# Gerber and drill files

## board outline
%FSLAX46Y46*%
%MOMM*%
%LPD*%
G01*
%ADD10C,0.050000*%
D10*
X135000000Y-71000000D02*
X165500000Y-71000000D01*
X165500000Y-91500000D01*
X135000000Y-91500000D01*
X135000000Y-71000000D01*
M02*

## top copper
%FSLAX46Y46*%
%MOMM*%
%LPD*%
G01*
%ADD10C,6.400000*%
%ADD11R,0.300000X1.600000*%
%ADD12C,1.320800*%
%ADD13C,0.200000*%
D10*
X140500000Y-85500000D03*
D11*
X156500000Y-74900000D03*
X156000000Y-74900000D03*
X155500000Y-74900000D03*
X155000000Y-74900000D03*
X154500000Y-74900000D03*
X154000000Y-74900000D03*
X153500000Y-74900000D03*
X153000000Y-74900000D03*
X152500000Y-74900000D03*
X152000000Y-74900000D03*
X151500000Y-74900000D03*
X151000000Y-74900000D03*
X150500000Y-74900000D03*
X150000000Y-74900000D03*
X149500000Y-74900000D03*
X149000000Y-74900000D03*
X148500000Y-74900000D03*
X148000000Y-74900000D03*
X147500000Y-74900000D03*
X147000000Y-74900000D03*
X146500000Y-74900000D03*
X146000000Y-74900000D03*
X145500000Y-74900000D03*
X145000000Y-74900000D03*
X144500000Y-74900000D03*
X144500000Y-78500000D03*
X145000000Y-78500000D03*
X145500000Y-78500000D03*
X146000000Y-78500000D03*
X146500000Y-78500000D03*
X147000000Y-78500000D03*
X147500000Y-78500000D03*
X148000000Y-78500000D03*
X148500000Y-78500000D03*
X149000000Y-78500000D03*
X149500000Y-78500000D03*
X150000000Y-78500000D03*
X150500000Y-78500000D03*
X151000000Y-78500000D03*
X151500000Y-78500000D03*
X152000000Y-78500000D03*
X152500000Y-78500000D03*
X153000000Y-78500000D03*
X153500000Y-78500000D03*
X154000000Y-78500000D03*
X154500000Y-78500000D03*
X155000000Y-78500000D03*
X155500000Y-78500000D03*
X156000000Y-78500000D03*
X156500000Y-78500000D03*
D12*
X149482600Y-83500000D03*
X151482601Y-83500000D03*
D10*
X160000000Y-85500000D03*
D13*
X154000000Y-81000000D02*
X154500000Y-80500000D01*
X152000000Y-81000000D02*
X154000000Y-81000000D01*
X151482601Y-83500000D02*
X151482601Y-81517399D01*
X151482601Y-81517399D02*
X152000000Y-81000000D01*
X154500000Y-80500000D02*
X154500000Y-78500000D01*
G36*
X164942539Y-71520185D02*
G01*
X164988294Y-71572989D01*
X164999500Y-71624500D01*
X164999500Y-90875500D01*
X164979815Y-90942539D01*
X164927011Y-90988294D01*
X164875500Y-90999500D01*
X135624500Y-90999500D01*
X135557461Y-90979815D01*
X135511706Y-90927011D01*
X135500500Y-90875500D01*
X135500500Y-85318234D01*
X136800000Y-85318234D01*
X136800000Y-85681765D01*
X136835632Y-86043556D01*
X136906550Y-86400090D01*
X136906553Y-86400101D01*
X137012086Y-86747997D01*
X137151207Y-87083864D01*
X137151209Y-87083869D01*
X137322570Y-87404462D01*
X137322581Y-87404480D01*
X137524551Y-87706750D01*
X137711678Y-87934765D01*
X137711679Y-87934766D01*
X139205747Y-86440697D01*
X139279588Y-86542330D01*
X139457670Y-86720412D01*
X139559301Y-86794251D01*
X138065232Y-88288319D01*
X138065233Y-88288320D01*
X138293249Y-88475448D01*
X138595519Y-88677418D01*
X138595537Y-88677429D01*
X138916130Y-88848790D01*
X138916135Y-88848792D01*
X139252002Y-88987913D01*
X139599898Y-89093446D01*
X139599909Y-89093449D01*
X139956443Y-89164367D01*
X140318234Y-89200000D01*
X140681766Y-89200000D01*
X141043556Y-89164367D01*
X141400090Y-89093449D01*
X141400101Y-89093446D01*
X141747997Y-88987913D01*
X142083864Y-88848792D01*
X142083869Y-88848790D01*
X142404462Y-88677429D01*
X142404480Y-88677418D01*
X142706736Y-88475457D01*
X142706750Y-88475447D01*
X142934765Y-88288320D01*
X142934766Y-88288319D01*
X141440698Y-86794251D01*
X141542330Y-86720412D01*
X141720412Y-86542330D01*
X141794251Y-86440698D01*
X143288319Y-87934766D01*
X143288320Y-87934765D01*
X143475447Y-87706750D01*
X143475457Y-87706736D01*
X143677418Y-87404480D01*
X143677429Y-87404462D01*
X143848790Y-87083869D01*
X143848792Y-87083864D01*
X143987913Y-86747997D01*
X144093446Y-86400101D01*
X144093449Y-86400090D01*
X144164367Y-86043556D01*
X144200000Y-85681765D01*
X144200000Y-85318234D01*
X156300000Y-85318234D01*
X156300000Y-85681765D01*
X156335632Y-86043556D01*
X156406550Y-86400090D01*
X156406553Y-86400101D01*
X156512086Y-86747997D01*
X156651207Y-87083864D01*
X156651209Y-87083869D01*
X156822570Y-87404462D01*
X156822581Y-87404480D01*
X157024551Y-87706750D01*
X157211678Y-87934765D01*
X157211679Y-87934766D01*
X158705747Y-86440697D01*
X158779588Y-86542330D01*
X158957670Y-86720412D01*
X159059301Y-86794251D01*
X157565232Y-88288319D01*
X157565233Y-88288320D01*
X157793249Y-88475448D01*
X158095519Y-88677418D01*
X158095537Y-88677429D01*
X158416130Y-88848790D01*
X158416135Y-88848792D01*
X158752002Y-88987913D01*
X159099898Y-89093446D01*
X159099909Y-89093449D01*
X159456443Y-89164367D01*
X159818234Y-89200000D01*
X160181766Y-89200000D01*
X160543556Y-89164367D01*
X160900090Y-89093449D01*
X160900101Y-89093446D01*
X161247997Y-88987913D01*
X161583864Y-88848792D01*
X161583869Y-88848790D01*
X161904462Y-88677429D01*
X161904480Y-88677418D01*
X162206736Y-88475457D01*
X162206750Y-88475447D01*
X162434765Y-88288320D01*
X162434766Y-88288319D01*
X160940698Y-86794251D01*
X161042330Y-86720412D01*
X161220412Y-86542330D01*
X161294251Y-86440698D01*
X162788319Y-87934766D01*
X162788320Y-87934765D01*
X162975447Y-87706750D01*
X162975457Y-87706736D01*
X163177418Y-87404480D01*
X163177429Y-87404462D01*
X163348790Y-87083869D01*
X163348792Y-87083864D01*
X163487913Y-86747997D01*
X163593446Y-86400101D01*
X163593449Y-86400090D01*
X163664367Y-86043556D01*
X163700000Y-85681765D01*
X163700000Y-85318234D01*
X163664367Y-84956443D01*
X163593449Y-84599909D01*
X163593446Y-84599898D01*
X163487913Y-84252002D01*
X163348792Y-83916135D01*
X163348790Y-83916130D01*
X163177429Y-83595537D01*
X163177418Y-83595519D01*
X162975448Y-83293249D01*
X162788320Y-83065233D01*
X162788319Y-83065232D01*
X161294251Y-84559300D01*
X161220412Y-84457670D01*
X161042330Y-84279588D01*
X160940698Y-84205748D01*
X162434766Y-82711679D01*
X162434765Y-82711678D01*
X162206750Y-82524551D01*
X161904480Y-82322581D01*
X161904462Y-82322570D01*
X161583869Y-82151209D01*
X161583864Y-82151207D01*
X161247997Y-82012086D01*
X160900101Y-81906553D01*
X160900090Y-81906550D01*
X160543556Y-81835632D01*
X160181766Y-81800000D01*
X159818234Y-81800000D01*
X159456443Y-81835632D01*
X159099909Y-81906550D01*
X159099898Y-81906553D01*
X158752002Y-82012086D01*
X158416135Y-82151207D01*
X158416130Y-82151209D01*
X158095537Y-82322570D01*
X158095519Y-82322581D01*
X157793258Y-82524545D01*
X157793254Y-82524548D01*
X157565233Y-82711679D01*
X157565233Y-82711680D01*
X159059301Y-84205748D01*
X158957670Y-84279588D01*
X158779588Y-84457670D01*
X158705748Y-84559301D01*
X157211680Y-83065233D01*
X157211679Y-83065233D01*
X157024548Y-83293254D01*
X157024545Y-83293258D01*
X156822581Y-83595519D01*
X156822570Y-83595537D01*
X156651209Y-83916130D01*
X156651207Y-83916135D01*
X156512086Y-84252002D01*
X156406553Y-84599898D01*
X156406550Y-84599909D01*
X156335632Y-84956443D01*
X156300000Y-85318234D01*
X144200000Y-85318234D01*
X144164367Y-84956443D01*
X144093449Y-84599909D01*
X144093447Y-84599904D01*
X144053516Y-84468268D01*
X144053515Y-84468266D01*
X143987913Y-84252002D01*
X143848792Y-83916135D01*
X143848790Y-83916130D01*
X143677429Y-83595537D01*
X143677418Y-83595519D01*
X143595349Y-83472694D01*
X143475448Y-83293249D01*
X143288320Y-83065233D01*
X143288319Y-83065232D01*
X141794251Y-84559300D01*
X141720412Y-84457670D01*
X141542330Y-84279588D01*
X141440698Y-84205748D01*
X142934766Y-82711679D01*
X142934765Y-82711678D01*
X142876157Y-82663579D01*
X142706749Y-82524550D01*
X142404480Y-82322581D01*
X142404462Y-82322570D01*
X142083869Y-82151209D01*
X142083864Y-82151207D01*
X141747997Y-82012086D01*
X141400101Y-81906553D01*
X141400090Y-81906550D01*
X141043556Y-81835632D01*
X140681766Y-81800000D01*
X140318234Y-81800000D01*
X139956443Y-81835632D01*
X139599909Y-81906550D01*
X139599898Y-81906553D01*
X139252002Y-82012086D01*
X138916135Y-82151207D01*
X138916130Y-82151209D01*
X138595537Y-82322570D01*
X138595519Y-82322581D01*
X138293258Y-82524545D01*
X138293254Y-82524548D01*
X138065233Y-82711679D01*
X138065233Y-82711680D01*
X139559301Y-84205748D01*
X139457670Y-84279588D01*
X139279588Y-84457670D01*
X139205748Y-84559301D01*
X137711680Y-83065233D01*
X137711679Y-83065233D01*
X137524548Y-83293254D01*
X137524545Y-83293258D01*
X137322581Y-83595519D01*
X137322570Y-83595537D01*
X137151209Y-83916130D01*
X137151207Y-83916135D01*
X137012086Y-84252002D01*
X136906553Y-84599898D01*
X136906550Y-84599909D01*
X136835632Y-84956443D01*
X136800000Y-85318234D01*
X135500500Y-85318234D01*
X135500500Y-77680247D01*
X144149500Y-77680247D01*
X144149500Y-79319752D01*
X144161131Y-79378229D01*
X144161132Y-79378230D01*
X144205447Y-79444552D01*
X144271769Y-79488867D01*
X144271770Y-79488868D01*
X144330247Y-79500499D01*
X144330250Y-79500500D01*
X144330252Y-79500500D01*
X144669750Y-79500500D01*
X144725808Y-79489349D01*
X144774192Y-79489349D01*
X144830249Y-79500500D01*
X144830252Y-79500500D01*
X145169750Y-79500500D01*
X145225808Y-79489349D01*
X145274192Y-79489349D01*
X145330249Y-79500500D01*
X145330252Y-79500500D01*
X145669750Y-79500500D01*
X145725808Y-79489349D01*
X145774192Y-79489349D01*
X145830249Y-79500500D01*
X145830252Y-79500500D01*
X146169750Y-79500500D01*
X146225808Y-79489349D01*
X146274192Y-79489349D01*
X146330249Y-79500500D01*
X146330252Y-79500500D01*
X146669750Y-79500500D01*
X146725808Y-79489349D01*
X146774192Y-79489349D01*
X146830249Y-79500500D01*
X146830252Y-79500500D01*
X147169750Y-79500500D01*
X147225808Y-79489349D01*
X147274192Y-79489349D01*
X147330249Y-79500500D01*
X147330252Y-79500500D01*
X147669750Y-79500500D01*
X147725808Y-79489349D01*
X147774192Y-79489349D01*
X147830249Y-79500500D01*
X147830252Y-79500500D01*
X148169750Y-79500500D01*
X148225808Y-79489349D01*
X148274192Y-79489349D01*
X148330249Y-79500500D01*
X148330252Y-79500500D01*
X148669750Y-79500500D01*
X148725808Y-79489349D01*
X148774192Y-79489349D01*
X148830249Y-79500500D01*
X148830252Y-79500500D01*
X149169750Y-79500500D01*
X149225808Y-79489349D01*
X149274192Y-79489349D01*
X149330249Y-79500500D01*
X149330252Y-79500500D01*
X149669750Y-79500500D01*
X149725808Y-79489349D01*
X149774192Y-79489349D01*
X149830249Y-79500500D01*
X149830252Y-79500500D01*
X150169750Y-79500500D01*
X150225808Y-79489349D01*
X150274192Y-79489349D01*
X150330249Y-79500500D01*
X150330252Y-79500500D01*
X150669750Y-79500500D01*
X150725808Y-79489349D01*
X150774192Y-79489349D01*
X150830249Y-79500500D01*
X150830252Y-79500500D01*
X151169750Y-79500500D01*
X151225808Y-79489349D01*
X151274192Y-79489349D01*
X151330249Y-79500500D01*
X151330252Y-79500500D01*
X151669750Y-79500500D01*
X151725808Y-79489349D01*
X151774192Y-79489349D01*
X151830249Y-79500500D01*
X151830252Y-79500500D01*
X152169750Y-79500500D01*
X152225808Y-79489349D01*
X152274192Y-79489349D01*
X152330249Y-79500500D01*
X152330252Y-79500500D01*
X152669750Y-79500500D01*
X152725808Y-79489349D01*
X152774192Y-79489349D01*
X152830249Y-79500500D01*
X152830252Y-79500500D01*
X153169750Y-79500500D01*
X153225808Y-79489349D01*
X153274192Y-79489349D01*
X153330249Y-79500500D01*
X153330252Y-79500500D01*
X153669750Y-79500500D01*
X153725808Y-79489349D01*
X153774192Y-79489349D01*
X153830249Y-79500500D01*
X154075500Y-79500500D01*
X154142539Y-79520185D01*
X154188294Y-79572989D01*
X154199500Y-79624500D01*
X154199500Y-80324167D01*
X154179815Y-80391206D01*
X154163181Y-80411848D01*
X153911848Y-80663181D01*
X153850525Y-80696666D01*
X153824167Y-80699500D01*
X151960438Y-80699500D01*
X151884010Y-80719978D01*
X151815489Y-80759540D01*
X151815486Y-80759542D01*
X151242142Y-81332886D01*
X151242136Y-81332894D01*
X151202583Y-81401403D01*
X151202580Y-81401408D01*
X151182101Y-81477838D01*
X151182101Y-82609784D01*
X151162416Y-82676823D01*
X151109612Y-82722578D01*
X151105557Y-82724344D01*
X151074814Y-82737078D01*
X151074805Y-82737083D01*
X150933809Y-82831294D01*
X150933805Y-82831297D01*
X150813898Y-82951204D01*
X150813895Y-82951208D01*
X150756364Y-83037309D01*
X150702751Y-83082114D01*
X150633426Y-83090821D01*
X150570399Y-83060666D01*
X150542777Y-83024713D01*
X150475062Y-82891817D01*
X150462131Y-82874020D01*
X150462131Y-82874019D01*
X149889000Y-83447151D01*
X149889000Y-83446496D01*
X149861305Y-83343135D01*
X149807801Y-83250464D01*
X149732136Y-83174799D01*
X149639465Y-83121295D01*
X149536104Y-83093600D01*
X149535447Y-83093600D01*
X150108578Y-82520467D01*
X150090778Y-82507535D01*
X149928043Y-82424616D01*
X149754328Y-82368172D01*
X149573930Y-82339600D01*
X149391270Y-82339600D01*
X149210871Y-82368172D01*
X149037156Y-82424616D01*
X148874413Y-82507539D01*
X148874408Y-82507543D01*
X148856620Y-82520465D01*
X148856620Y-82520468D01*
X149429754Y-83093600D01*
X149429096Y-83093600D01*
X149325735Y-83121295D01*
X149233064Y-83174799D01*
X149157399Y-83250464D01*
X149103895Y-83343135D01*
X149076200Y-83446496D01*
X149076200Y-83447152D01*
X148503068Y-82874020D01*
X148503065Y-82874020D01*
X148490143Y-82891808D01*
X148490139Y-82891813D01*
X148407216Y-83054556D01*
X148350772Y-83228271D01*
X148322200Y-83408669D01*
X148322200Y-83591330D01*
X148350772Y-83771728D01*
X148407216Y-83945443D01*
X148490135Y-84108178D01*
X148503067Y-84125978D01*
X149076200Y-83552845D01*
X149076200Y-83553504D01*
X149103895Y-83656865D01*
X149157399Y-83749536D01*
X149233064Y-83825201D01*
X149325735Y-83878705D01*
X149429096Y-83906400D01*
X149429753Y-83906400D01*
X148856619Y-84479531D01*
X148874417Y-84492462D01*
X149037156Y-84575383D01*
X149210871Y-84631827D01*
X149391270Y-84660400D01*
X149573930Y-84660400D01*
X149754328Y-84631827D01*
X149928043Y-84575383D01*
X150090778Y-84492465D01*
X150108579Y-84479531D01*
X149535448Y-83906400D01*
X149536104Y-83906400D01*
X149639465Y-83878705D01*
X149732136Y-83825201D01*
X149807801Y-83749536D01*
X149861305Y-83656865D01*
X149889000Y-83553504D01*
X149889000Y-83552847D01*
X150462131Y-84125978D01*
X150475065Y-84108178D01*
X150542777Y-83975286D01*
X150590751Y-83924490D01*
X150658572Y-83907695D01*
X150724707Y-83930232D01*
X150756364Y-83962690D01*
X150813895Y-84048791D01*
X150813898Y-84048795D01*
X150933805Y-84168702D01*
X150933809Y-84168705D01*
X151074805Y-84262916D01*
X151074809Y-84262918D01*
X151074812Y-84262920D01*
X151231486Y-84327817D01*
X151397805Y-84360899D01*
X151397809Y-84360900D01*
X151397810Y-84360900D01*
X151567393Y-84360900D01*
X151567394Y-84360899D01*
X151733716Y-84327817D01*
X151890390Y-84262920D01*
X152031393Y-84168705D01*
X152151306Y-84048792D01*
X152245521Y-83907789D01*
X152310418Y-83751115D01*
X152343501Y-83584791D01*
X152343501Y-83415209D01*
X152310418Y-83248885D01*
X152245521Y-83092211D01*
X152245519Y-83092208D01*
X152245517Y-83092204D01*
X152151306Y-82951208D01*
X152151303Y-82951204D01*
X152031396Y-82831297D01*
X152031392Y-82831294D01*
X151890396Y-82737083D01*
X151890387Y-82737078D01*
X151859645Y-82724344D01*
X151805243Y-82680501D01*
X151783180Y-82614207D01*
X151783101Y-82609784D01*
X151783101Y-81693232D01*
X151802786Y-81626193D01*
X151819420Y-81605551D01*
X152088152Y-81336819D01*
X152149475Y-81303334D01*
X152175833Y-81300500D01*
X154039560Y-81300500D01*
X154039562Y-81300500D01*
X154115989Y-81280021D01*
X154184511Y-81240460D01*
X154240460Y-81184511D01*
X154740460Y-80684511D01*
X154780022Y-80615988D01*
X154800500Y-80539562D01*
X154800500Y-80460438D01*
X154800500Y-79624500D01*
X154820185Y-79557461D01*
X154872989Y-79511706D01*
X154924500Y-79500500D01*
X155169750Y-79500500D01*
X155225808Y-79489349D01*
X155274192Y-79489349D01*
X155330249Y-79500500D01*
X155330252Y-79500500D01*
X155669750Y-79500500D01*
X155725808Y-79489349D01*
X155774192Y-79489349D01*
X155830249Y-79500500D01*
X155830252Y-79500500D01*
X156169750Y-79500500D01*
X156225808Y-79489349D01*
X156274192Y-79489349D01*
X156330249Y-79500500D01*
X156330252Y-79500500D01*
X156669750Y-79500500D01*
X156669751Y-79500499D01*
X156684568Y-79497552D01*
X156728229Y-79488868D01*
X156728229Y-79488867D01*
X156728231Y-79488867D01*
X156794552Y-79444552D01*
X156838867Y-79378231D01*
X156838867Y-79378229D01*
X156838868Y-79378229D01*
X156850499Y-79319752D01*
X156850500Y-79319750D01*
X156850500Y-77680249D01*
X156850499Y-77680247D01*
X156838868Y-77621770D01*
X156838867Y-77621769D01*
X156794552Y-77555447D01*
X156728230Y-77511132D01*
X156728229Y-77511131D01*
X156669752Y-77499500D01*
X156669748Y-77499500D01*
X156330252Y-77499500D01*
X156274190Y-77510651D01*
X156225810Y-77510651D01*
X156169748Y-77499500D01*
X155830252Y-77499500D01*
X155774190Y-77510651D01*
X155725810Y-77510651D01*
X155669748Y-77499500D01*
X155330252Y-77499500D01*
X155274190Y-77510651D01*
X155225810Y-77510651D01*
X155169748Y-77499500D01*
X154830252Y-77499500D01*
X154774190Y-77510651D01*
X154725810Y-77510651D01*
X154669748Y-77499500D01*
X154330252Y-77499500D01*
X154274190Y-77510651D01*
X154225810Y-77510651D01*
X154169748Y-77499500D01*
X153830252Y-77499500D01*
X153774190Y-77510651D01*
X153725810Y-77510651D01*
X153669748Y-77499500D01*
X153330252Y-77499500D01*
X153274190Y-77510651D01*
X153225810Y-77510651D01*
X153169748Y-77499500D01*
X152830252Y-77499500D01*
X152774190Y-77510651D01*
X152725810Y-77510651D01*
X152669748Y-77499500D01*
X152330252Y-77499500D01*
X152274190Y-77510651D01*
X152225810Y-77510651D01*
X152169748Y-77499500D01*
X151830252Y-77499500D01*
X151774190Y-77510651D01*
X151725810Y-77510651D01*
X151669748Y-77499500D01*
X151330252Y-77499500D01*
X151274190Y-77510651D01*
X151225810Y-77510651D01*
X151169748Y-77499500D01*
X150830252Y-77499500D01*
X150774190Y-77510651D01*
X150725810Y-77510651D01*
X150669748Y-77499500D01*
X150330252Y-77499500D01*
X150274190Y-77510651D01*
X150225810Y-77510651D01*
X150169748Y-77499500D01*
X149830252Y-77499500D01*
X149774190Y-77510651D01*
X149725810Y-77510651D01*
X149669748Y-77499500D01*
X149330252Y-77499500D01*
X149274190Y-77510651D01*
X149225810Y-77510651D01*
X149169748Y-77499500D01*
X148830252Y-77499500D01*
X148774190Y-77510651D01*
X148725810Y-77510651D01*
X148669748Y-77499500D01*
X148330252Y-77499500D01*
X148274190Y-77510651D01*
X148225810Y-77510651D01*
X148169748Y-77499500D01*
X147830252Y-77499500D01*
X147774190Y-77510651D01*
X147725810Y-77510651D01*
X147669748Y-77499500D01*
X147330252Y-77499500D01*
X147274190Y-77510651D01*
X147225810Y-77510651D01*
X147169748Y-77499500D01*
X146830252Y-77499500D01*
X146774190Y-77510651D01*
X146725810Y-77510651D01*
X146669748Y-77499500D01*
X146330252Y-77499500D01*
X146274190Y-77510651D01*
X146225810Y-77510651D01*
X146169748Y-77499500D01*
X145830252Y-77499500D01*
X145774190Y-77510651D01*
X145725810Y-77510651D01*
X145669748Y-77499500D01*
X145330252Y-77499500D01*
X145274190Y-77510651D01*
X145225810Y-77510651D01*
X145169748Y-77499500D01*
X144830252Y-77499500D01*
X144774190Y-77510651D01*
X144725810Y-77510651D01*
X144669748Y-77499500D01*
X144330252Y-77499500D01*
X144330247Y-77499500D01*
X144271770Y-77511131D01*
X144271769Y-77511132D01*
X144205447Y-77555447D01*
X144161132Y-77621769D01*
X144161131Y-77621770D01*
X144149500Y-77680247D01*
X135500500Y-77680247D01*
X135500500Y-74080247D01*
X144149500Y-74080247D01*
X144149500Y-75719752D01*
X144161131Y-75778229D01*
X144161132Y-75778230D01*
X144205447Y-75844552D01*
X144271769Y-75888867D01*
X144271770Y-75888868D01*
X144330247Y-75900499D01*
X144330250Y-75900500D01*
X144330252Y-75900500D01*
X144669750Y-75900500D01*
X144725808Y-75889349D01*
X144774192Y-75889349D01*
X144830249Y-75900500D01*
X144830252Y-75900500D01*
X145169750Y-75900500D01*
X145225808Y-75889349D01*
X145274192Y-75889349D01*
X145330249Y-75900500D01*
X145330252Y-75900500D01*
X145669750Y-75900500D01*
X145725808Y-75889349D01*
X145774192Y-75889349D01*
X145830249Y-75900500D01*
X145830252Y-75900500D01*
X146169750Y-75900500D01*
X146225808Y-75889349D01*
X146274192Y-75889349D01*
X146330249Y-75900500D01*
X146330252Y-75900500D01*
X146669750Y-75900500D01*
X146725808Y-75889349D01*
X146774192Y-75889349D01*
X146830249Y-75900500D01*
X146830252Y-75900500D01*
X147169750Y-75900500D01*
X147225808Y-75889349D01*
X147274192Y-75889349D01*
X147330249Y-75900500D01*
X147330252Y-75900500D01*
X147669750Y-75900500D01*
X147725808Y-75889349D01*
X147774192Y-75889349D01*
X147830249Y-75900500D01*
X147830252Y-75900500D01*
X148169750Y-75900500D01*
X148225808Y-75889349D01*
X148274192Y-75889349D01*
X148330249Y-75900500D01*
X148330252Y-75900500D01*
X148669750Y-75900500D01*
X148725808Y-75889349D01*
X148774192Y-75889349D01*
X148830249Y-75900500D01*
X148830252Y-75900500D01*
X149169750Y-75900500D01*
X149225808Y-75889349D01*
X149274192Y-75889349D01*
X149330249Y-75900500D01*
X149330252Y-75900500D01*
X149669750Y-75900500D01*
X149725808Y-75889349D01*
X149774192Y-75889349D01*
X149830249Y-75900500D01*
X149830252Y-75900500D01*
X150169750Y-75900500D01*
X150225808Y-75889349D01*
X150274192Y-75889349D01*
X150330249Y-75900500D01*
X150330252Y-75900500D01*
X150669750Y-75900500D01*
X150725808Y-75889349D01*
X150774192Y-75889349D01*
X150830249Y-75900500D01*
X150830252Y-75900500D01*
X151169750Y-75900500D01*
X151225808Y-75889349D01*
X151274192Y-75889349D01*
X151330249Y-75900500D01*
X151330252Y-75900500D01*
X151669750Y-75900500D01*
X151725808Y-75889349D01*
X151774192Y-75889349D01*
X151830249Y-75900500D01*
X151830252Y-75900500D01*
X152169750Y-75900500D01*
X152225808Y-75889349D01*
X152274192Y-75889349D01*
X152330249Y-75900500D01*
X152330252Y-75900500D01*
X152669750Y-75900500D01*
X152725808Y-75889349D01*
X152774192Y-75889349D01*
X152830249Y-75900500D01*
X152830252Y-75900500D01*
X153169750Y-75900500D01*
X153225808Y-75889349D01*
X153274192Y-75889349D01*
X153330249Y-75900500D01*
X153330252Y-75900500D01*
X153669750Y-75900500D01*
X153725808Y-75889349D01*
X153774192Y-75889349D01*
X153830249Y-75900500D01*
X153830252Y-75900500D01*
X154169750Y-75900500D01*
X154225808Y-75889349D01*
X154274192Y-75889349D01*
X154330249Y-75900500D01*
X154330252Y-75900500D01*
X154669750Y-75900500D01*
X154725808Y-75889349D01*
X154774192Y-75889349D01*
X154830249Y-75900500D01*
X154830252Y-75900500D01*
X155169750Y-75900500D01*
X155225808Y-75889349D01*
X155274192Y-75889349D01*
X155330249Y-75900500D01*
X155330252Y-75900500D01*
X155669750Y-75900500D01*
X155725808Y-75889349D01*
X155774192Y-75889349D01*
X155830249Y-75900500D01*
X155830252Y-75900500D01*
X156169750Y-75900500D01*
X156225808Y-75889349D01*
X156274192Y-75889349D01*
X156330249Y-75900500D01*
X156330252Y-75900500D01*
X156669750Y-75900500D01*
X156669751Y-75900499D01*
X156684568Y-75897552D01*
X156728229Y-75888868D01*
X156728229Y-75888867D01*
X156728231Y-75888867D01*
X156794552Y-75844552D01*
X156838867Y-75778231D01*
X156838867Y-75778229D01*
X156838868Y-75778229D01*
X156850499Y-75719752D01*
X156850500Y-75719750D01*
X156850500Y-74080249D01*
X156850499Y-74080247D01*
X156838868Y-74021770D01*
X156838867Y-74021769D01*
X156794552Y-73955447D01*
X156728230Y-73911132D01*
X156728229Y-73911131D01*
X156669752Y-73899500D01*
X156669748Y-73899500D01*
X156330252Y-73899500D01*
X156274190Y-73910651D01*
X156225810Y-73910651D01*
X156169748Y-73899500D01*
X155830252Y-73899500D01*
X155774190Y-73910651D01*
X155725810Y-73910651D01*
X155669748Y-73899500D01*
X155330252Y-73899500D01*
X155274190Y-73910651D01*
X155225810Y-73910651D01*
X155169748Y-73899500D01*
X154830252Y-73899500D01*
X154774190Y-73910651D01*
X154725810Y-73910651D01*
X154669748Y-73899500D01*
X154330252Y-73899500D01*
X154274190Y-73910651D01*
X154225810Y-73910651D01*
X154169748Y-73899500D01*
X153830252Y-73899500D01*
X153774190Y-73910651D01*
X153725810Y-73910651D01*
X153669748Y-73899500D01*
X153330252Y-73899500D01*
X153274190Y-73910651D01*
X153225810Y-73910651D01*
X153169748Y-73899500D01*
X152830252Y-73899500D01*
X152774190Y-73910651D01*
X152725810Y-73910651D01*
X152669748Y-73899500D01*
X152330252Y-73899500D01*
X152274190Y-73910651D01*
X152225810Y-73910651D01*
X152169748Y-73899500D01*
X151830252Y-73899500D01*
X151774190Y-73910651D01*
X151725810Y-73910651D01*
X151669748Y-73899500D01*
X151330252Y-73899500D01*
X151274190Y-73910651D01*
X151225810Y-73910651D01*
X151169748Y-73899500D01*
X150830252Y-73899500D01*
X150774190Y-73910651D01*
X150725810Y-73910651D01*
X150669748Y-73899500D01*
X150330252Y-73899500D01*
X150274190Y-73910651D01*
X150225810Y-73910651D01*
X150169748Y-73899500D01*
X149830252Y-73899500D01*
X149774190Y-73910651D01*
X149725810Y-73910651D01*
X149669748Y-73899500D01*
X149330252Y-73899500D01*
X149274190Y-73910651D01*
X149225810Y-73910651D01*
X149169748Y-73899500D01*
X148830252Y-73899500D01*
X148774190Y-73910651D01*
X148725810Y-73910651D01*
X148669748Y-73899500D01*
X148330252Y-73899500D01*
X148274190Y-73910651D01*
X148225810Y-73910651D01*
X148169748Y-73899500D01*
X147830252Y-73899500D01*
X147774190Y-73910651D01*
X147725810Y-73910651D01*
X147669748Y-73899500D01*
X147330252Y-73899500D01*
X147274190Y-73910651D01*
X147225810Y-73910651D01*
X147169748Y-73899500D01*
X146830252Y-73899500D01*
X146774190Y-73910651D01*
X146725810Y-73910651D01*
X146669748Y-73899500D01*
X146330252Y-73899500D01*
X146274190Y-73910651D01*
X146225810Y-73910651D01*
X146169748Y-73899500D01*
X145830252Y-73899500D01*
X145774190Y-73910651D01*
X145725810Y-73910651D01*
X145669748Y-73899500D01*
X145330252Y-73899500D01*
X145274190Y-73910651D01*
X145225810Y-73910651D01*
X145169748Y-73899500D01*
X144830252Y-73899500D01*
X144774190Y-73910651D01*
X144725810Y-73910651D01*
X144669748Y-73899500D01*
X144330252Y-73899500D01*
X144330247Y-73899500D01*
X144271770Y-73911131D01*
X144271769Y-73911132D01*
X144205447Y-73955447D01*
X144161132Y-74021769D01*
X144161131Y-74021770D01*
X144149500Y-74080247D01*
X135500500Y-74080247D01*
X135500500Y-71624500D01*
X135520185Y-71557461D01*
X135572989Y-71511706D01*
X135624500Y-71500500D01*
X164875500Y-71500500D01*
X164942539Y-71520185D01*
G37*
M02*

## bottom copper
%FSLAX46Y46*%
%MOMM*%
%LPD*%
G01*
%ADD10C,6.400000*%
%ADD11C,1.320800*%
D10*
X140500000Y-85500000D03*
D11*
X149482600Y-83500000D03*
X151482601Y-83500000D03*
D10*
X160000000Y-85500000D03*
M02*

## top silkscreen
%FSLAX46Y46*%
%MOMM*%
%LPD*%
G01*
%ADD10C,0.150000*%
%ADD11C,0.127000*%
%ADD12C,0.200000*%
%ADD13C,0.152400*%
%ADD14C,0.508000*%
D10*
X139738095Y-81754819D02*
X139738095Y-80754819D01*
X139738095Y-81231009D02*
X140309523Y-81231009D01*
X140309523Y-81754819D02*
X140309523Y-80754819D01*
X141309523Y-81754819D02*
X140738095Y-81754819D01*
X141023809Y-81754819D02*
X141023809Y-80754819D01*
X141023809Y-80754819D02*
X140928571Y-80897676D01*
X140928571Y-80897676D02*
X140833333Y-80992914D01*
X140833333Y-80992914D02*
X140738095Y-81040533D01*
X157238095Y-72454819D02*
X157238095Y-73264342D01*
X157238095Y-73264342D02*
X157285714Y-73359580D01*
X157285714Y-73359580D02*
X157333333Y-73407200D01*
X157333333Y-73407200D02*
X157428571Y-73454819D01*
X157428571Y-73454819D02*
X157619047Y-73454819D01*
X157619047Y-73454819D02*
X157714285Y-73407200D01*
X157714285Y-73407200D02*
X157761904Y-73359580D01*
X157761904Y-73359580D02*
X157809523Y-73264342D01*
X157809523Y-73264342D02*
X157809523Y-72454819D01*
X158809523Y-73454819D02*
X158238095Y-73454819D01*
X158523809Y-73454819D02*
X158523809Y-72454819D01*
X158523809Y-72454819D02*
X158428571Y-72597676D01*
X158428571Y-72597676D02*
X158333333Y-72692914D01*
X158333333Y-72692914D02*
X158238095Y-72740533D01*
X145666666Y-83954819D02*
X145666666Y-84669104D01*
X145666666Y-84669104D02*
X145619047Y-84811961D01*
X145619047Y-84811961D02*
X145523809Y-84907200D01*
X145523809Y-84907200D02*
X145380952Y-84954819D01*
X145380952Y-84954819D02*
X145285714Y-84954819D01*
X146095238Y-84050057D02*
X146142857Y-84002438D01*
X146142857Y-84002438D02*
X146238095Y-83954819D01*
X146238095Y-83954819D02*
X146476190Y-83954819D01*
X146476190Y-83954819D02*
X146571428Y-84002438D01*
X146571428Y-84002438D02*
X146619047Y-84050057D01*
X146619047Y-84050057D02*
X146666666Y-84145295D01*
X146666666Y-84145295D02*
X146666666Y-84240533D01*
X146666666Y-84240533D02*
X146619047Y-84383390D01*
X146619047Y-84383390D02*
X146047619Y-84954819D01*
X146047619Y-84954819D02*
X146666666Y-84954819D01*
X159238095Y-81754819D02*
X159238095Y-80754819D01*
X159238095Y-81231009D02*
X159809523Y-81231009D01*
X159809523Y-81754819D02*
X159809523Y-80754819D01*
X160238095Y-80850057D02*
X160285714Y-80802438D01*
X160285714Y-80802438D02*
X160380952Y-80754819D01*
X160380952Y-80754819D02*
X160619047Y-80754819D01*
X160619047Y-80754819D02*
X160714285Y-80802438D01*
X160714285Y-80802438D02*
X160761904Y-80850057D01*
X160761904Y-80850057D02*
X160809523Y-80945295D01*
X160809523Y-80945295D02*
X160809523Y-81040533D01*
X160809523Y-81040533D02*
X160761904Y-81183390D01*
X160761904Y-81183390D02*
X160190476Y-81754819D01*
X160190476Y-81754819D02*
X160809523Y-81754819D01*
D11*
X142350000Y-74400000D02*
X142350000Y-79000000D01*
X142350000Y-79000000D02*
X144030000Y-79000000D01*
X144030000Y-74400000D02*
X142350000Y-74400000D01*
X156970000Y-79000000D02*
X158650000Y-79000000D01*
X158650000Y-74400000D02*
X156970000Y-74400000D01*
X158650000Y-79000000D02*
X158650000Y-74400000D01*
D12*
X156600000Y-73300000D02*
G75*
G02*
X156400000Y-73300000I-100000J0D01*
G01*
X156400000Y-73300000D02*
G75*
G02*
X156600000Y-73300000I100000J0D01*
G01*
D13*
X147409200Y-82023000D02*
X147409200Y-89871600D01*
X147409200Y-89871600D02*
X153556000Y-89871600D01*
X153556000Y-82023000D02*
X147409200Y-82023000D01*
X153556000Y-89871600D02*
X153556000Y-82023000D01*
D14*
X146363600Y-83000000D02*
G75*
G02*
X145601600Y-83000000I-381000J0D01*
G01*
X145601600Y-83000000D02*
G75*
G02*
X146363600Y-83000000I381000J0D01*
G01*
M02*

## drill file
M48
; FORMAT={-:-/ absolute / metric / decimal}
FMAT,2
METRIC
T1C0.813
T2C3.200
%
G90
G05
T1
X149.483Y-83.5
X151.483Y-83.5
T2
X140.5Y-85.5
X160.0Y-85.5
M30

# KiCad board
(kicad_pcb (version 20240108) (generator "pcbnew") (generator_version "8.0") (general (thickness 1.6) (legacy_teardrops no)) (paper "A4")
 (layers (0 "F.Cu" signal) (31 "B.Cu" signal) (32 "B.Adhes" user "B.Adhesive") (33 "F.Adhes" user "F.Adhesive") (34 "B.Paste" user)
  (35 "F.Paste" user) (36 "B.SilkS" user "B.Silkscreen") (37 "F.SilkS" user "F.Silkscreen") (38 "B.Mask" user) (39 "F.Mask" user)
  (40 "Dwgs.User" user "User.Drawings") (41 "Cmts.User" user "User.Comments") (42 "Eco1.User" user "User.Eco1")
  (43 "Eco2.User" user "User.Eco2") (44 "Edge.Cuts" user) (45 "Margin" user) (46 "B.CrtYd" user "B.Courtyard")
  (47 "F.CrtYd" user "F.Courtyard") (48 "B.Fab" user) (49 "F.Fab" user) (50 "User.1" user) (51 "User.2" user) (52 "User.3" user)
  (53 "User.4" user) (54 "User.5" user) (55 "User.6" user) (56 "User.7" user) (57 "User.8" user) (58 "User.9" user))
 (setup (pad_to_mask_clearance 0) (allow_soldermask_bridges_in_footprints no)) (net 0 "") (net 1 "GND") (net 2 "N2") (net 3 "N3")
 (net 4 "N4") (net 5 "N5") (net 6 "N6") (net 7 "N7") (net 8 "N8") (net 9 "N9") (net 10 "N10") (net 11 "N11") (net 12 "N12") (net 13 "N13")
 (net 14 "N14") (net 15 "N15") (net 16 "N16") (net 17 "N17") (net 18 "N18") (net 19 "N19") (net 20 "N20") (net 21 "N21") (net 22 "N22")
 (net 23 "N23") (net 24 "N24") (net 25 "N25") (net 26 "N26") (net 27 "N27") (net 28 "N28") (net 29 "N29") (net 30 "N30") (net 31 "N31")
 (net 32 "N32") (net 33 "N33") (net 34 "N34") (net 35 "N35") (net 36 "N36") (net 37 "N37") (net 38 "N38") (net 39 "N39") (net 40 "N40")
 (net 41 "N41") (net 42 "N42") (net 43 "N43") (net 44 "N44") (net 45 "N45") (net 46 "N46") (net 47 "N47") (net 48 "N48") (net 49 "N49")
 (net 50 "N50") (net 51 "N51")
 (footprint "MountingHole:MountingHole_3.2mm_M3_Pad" (layer "F.Cu") (at 140.5 85.5)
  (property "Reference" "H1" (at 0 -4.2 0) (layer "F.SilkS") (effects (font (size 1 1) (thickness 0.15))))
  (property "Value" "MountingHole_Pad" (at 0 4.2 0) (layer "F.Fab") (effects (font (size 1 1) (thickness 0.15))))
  (pad "1" thru_hole circle (at 0 0) (size 6.4 6.4) (drill 3.2) (layers "*.Cu" "*.Mask") (remove_unused_layers no) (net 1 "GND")))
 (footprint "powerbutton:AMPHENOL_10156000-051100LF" (layer "F.Cu") (at 150.5 76.7)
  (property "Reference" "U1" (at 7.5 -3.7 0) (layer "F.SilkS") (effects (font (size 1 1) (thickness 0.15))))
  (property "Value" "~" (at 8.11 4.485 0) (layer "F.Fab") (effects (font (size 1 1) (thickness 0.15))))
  (fp_line (start -8.15 -2.3) (end -8.15 2.3) (stroke (width 0.127) (type solid)) (layer "F.SilkS"))
  (fp_line (start -8.15 2.3) (end -6.47 2.3) (stroke (width 0.127) (type solid)) (layer "F.SilkS"))
  (fp_line (start -6.47 -2.3) (end -8.15 -2.3) (stroke (width 0.127) (type solid)) (layer "F.SilkS"))
  (fp_line (start 6.47 2.3) (end 8.15 2.3) (stroke (width 0.127) (type solid)) (layer "F.SilkS"))
  (fp_line (start 8.15 -2.3) (end 6.47 -2.3) (stroke (width 0.127) (type solid)) (layer "F.SilkS"))
  (fp_line (start 8.15 2.3) (end 8.15 -2.3) (stroke (width 0.127) (type solid)) (layer "F.SilkS"))
  (fp_circle (center 6 -3.4) (end 6.1 -3.4) (stroke (width 0.2) (type solid)) (fill none) (layer "F.SilkS"))
  (pad "1" smd rect (at 6 -1.8) (size 0.3 1.6) (layers "F.Cu" "F.Paste") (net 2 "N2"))
  (pad "2" smd rect (at 5.5 -1.8) (size 0.3 1.6) (layers "F.Cu" "F.Paste") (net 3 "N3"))
  (pad "3" smd rect (at 5 -1.8) (size 0.3 1.6) (layers "F.Cu" "F.Paste") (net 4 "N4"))
  (pad "4" smd rect (at 4.5 -1.8) (size 0.3 1.6) (layers "F.Cu" "F.Paste") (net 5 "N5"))
  (pad "5" smd rect (at 4 -1.8) (size 0.3 1.6) (layers "F.Cu" "F.Paste") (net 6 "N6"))
  (pad "6" smd rect (at 3.5 -1.8) (size 0.3 1.6) (layers "F.Cu" "F.Paste") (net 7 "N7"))
  (pad "7" smd rect (at 3 -1.8) (size 0.3 1.6) (layers "F.Cu" "F.Paste") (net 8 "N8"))
  (pad "8" smd rect (at 2.5 -1.8) (size 0.3 1.6) (layers "F.Cu" "F.Paste") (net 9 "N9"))
  (pad "9" smd rect (at 2 -1.8) (size 0.3 1.6) (layers "F.Cu" "F.Paste") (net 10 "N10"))
  (pad "10" smd rect (at 1.5 -1.8) (size 0.3 1.6) (layers "F.Cu" "F.Paste") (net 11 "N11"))
  (pad "11" smd rect (at 1 -1.8) (size 0.3 1.6) (layers "F.Cu" "F.Paste") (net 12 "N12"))
  (pad "12" smd rect (at 0.5 -1.8) (size 0.3 1.6) (layers "F.Cu" "F.Paste") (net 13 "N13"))
  (pad "13" smd rect (at 0 -1.8) (size 0.3 1.6) (layers "F.Cu" "F.Paste") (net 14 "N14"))
  (pad "14" smd rect (at -0.5 -1.8) (size 0.3 1.6) (layers "F.Cu" "F.Paste") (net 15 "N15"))
  (pad "15" smd rect (at -1 -1.8) (size 0.3 1.6) (layers "F.Cu" "F.Paste") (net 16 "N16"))
  (pad "16" smd rect (at -1.5 -1.8) (size 0.3 1.6) (layers "F.Cu" "F.Paste") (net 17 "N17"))
  (pad "17" smd rect (at -2 -1.8) (size 0.3 1.6) (layers "F.Cu" "F.Paste") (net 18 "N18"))
  (pad "18" smd rect (at -2.5 -1.8) (size 0.3 1.6) (layers "F.Cu" "F.Paste") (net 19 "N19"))
  (pad "19" smd rect (at -3 -1.8) (size 0.3 1.6) (layers "F.Cu" "F.Paste") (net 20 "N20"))
  (pad "20" smd rect (at -3.5 -1.8) (size 0.3 1.6) (layers "F.Cu" "F.Paste") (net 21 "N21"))
  (pad "21" smd rect (at -4 -1.8) (size 0.3 1.6) (layers "F.Cu" "F.Paste") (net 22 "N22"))
  (pad "22" smd rect (at -4.5 -1.8) (size 0.3 1.6) (layers "F.Cu" "F.Paste") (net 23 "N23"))
  (pad "23" smd rect (at -5 -1.8) (size 0.3 1.6) (layers "F.Cu" "F.Paste") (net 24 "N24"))
  (pad "24" smd rect (at -5.5 -1.8) (size 0.3 1.6) (layers "F.Cu" "F.Paste") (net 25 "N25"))
  (pad "25" smd rect (at -6 -1.8) (size 0.3 1.6) (layers "F.Cu" "F.Paste") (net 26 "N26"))
  (pad "26" smd rect (at -6 1.8) (size 0.3 1.6) (layers "F.Cu" "F.Paste") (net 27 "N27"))
  (pad "27" smd rect (at -5.5 1.8) (size 0.3 1.6) (layers "F.Cu" "F.Paste") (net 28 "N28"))
  (pad "28" smd rect (at -5 1.8) (size 0.3 1.6) (layers "F.Cu" "F.Paste") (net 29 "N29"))
  (pad "29" smd rect (at -4.5 1.8) (size 0.3 1.6) (layers "F.Cu" "F.Paste") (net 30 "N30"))
  (pad "30" smd rect (at -4 1.8) (size 0.3 1.6) (layers "F.Cu" "F.Paste") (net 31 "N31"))
  (pad "31" smd rect (at -3.5 1.8) (size 0.3 1.6) (layers "F.Cu" "F.Paste") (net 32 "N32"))
  (pad "32" smd rect (at -3 1.8) (size 0.3 1.6) (layers "F.Cu" "F.Paste") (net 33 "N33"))
  (pad "33" smd rect (at -2.5 1.8) (size 0.3 1.6) (layers "F.Cu" "F.Paste") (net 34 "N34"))
  (pad "34" smd rect (at -2 1.8) (size 0.3 1.6) (layers "F.Cu" "F.Paste") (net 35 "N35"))
  (pad "35" smd rect (at -1.5 1.8) (size 0.3 1.6) (layers "F.Cu" "F.Paste") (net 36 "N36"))
  (pad "36" smd rect (at -1 1.8) (size 0.3 1.6) (layers "F.Cu" "F.Paste") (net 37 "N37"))
  (pad "37" smd rect (at -0.5 1.8) (size 0.3 1.6) (layers "F.Cu" "F.Paste") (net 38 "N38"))
  (pad "38" smd rect (at 0 1.8) (size 0.3 1.6) (layers "F.Cu" "F.Paste") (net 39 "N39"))
  (pad "39" smd rect (at 0.5 1.8) (size 0.3 1.6) (layers "F.Cu" "F.Paste") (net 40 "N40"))
  (pad "40" smd rect (at 1 1.8) (size 0.3 1.6) (layers "F.Cu" "F.Paste") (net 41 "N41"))
  (pad "41" smd rect (at 1.5 1.8) (size 0.3 1.6) (layers "F.Cu" "F.Paste") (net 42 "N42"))
  (pad "42" smd rect (at 2 1.8) (size 0.3 1.6) (layers "F.Cu" "F.Paste") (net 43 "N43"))
  (pad "43" smd rect (at 2.5 1.8) (size 0.3 1.6) (layers "F.Cu" "F.Paste") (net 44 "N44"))
  (pad "44" smd rect (at 3 1.8) (size 0.3 1.6) (layers "F.Cu" "F.Paste") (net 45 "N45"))
  (pad "45" smd rect (at 3.5 1.8) (size 0.3 1.6) (layers "F.Cu" "F.Paste") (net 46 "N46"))
  (pad "46" smd rect (at 4 1.8) (size 0.3 1.6) (layers "F.Cu" "F.Paste") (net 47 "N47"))
  (pad "47" smd rect (at 4.5 1.8) (size 0.3 1.6) (layers "F.Cu" "F.Paste") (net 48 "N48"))
  (pad "48" smd rect (at 5 1.8) (size 0.3 1.6) (layers "F.Cu" "F.Paste") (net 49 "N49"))
  (pad "49" smd rect (at 5.5 1.8) (size 0.3 1.6) (layers "F.Cu" "F.Paste") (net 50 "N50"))
  (pad "50" smd rect (at 6 1.8) (size 0.3 1.6) (layers "F.Cu" "F.Paste") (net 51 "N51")))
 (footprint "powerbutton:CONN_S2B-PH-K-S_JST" (layer "F.Cu") (at 149.4826 83.5)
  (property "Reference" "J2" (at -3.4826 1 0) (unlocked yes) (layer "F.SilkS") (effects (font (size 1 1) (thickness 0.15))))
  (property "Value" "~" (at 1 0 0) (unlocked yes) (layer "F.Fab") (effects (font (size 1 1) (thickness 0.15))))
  (fp_line (start -2.0734 -1.477) (end -2.0734 6.3716) (stroke (width 0.1524) (type solid)) (layer "F.SilkS"))
  (fp_line (start -2.0734 6.3716) (end 4.0734 6.3716) (stroke (width 0.1524) (type solid)) (layer "F.SilkS"))
  (fp_line (start 4.0734 -1.477) (end -2.0734 -1.477) (stroke (width 0.1524) (type solid)) (layer "F.SilkS"))
  (fp_line (start 4.0734 6.3716) (end 4.0734 -1.477) (stroke (width 0.1524) (type solid)) (layer "F.SilkS"))
  (fp_circle (center -3.5 -0.5) (end -3.119 -0.5) (stroke (width 0.508) (type solid)) (fill none) (layer "F.SilkS"))
  (pad "1" thru_hole circle (at 0 0) (size 1.3208 1.3208) (drill 0.8128) (layers "*.Cu" "*.Mask") (remove_unused_layers no) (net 1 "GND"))
  (pad "2" thru_hole circle (at 2.000001 0) (size 1.3208 1.3208) (drill 0.8128) (layers "*.Cu" "*.Mask") (remove_unused_layers no)
   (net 47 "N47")))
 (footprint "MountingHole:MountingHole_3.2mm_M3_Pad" (layer "F.Cu") (at 160 85.5)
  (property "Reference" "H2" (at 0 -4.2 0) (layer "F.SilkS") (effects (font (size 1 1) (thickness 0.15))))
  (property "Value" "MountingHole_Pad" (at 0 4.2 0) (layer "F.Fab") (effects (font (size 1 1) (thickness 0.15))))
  (pad "1" thru_hole circle (at 0 0) (size 6.4 6.4) (drill 3.2) (layers "*.Cu" "*.Mask") (remove_unused_layers no) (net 1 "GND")))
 (gr_rect (start 135 71) (end 165.5 91.5) (stroke (width 0.05) (type default)) (fill none) (layer "Edge.Cuts"))
 (segment (start 154 81) (end 154.5 80.5) (width 0.2) (layer "F.Cu") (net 47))
 (segment (start 152 81) (end 154 81) (width 0.2) (layer "F.Cu") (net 47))
 (segment (start 151.482601 83.5) (end 151.482601 81.517399) (width 0.2) (layer "F.Cu") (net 47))
 (segment (start 151.482601 81.517399) (end 152 81) (width 0.2) (layer "F.Cu") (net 47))
 (segment (start 154.5 80.5) (end 154.5 78.5) (width 0.2) (layer "F.Cu") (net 47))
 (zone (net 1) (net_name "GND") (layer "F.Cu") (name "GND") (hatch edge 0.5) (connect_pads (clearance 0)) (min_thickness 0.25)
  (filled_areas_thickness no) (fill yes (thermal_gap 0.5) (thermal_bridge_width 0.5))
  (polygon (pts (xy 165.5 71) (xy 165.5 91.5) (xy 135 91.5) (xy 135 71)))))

